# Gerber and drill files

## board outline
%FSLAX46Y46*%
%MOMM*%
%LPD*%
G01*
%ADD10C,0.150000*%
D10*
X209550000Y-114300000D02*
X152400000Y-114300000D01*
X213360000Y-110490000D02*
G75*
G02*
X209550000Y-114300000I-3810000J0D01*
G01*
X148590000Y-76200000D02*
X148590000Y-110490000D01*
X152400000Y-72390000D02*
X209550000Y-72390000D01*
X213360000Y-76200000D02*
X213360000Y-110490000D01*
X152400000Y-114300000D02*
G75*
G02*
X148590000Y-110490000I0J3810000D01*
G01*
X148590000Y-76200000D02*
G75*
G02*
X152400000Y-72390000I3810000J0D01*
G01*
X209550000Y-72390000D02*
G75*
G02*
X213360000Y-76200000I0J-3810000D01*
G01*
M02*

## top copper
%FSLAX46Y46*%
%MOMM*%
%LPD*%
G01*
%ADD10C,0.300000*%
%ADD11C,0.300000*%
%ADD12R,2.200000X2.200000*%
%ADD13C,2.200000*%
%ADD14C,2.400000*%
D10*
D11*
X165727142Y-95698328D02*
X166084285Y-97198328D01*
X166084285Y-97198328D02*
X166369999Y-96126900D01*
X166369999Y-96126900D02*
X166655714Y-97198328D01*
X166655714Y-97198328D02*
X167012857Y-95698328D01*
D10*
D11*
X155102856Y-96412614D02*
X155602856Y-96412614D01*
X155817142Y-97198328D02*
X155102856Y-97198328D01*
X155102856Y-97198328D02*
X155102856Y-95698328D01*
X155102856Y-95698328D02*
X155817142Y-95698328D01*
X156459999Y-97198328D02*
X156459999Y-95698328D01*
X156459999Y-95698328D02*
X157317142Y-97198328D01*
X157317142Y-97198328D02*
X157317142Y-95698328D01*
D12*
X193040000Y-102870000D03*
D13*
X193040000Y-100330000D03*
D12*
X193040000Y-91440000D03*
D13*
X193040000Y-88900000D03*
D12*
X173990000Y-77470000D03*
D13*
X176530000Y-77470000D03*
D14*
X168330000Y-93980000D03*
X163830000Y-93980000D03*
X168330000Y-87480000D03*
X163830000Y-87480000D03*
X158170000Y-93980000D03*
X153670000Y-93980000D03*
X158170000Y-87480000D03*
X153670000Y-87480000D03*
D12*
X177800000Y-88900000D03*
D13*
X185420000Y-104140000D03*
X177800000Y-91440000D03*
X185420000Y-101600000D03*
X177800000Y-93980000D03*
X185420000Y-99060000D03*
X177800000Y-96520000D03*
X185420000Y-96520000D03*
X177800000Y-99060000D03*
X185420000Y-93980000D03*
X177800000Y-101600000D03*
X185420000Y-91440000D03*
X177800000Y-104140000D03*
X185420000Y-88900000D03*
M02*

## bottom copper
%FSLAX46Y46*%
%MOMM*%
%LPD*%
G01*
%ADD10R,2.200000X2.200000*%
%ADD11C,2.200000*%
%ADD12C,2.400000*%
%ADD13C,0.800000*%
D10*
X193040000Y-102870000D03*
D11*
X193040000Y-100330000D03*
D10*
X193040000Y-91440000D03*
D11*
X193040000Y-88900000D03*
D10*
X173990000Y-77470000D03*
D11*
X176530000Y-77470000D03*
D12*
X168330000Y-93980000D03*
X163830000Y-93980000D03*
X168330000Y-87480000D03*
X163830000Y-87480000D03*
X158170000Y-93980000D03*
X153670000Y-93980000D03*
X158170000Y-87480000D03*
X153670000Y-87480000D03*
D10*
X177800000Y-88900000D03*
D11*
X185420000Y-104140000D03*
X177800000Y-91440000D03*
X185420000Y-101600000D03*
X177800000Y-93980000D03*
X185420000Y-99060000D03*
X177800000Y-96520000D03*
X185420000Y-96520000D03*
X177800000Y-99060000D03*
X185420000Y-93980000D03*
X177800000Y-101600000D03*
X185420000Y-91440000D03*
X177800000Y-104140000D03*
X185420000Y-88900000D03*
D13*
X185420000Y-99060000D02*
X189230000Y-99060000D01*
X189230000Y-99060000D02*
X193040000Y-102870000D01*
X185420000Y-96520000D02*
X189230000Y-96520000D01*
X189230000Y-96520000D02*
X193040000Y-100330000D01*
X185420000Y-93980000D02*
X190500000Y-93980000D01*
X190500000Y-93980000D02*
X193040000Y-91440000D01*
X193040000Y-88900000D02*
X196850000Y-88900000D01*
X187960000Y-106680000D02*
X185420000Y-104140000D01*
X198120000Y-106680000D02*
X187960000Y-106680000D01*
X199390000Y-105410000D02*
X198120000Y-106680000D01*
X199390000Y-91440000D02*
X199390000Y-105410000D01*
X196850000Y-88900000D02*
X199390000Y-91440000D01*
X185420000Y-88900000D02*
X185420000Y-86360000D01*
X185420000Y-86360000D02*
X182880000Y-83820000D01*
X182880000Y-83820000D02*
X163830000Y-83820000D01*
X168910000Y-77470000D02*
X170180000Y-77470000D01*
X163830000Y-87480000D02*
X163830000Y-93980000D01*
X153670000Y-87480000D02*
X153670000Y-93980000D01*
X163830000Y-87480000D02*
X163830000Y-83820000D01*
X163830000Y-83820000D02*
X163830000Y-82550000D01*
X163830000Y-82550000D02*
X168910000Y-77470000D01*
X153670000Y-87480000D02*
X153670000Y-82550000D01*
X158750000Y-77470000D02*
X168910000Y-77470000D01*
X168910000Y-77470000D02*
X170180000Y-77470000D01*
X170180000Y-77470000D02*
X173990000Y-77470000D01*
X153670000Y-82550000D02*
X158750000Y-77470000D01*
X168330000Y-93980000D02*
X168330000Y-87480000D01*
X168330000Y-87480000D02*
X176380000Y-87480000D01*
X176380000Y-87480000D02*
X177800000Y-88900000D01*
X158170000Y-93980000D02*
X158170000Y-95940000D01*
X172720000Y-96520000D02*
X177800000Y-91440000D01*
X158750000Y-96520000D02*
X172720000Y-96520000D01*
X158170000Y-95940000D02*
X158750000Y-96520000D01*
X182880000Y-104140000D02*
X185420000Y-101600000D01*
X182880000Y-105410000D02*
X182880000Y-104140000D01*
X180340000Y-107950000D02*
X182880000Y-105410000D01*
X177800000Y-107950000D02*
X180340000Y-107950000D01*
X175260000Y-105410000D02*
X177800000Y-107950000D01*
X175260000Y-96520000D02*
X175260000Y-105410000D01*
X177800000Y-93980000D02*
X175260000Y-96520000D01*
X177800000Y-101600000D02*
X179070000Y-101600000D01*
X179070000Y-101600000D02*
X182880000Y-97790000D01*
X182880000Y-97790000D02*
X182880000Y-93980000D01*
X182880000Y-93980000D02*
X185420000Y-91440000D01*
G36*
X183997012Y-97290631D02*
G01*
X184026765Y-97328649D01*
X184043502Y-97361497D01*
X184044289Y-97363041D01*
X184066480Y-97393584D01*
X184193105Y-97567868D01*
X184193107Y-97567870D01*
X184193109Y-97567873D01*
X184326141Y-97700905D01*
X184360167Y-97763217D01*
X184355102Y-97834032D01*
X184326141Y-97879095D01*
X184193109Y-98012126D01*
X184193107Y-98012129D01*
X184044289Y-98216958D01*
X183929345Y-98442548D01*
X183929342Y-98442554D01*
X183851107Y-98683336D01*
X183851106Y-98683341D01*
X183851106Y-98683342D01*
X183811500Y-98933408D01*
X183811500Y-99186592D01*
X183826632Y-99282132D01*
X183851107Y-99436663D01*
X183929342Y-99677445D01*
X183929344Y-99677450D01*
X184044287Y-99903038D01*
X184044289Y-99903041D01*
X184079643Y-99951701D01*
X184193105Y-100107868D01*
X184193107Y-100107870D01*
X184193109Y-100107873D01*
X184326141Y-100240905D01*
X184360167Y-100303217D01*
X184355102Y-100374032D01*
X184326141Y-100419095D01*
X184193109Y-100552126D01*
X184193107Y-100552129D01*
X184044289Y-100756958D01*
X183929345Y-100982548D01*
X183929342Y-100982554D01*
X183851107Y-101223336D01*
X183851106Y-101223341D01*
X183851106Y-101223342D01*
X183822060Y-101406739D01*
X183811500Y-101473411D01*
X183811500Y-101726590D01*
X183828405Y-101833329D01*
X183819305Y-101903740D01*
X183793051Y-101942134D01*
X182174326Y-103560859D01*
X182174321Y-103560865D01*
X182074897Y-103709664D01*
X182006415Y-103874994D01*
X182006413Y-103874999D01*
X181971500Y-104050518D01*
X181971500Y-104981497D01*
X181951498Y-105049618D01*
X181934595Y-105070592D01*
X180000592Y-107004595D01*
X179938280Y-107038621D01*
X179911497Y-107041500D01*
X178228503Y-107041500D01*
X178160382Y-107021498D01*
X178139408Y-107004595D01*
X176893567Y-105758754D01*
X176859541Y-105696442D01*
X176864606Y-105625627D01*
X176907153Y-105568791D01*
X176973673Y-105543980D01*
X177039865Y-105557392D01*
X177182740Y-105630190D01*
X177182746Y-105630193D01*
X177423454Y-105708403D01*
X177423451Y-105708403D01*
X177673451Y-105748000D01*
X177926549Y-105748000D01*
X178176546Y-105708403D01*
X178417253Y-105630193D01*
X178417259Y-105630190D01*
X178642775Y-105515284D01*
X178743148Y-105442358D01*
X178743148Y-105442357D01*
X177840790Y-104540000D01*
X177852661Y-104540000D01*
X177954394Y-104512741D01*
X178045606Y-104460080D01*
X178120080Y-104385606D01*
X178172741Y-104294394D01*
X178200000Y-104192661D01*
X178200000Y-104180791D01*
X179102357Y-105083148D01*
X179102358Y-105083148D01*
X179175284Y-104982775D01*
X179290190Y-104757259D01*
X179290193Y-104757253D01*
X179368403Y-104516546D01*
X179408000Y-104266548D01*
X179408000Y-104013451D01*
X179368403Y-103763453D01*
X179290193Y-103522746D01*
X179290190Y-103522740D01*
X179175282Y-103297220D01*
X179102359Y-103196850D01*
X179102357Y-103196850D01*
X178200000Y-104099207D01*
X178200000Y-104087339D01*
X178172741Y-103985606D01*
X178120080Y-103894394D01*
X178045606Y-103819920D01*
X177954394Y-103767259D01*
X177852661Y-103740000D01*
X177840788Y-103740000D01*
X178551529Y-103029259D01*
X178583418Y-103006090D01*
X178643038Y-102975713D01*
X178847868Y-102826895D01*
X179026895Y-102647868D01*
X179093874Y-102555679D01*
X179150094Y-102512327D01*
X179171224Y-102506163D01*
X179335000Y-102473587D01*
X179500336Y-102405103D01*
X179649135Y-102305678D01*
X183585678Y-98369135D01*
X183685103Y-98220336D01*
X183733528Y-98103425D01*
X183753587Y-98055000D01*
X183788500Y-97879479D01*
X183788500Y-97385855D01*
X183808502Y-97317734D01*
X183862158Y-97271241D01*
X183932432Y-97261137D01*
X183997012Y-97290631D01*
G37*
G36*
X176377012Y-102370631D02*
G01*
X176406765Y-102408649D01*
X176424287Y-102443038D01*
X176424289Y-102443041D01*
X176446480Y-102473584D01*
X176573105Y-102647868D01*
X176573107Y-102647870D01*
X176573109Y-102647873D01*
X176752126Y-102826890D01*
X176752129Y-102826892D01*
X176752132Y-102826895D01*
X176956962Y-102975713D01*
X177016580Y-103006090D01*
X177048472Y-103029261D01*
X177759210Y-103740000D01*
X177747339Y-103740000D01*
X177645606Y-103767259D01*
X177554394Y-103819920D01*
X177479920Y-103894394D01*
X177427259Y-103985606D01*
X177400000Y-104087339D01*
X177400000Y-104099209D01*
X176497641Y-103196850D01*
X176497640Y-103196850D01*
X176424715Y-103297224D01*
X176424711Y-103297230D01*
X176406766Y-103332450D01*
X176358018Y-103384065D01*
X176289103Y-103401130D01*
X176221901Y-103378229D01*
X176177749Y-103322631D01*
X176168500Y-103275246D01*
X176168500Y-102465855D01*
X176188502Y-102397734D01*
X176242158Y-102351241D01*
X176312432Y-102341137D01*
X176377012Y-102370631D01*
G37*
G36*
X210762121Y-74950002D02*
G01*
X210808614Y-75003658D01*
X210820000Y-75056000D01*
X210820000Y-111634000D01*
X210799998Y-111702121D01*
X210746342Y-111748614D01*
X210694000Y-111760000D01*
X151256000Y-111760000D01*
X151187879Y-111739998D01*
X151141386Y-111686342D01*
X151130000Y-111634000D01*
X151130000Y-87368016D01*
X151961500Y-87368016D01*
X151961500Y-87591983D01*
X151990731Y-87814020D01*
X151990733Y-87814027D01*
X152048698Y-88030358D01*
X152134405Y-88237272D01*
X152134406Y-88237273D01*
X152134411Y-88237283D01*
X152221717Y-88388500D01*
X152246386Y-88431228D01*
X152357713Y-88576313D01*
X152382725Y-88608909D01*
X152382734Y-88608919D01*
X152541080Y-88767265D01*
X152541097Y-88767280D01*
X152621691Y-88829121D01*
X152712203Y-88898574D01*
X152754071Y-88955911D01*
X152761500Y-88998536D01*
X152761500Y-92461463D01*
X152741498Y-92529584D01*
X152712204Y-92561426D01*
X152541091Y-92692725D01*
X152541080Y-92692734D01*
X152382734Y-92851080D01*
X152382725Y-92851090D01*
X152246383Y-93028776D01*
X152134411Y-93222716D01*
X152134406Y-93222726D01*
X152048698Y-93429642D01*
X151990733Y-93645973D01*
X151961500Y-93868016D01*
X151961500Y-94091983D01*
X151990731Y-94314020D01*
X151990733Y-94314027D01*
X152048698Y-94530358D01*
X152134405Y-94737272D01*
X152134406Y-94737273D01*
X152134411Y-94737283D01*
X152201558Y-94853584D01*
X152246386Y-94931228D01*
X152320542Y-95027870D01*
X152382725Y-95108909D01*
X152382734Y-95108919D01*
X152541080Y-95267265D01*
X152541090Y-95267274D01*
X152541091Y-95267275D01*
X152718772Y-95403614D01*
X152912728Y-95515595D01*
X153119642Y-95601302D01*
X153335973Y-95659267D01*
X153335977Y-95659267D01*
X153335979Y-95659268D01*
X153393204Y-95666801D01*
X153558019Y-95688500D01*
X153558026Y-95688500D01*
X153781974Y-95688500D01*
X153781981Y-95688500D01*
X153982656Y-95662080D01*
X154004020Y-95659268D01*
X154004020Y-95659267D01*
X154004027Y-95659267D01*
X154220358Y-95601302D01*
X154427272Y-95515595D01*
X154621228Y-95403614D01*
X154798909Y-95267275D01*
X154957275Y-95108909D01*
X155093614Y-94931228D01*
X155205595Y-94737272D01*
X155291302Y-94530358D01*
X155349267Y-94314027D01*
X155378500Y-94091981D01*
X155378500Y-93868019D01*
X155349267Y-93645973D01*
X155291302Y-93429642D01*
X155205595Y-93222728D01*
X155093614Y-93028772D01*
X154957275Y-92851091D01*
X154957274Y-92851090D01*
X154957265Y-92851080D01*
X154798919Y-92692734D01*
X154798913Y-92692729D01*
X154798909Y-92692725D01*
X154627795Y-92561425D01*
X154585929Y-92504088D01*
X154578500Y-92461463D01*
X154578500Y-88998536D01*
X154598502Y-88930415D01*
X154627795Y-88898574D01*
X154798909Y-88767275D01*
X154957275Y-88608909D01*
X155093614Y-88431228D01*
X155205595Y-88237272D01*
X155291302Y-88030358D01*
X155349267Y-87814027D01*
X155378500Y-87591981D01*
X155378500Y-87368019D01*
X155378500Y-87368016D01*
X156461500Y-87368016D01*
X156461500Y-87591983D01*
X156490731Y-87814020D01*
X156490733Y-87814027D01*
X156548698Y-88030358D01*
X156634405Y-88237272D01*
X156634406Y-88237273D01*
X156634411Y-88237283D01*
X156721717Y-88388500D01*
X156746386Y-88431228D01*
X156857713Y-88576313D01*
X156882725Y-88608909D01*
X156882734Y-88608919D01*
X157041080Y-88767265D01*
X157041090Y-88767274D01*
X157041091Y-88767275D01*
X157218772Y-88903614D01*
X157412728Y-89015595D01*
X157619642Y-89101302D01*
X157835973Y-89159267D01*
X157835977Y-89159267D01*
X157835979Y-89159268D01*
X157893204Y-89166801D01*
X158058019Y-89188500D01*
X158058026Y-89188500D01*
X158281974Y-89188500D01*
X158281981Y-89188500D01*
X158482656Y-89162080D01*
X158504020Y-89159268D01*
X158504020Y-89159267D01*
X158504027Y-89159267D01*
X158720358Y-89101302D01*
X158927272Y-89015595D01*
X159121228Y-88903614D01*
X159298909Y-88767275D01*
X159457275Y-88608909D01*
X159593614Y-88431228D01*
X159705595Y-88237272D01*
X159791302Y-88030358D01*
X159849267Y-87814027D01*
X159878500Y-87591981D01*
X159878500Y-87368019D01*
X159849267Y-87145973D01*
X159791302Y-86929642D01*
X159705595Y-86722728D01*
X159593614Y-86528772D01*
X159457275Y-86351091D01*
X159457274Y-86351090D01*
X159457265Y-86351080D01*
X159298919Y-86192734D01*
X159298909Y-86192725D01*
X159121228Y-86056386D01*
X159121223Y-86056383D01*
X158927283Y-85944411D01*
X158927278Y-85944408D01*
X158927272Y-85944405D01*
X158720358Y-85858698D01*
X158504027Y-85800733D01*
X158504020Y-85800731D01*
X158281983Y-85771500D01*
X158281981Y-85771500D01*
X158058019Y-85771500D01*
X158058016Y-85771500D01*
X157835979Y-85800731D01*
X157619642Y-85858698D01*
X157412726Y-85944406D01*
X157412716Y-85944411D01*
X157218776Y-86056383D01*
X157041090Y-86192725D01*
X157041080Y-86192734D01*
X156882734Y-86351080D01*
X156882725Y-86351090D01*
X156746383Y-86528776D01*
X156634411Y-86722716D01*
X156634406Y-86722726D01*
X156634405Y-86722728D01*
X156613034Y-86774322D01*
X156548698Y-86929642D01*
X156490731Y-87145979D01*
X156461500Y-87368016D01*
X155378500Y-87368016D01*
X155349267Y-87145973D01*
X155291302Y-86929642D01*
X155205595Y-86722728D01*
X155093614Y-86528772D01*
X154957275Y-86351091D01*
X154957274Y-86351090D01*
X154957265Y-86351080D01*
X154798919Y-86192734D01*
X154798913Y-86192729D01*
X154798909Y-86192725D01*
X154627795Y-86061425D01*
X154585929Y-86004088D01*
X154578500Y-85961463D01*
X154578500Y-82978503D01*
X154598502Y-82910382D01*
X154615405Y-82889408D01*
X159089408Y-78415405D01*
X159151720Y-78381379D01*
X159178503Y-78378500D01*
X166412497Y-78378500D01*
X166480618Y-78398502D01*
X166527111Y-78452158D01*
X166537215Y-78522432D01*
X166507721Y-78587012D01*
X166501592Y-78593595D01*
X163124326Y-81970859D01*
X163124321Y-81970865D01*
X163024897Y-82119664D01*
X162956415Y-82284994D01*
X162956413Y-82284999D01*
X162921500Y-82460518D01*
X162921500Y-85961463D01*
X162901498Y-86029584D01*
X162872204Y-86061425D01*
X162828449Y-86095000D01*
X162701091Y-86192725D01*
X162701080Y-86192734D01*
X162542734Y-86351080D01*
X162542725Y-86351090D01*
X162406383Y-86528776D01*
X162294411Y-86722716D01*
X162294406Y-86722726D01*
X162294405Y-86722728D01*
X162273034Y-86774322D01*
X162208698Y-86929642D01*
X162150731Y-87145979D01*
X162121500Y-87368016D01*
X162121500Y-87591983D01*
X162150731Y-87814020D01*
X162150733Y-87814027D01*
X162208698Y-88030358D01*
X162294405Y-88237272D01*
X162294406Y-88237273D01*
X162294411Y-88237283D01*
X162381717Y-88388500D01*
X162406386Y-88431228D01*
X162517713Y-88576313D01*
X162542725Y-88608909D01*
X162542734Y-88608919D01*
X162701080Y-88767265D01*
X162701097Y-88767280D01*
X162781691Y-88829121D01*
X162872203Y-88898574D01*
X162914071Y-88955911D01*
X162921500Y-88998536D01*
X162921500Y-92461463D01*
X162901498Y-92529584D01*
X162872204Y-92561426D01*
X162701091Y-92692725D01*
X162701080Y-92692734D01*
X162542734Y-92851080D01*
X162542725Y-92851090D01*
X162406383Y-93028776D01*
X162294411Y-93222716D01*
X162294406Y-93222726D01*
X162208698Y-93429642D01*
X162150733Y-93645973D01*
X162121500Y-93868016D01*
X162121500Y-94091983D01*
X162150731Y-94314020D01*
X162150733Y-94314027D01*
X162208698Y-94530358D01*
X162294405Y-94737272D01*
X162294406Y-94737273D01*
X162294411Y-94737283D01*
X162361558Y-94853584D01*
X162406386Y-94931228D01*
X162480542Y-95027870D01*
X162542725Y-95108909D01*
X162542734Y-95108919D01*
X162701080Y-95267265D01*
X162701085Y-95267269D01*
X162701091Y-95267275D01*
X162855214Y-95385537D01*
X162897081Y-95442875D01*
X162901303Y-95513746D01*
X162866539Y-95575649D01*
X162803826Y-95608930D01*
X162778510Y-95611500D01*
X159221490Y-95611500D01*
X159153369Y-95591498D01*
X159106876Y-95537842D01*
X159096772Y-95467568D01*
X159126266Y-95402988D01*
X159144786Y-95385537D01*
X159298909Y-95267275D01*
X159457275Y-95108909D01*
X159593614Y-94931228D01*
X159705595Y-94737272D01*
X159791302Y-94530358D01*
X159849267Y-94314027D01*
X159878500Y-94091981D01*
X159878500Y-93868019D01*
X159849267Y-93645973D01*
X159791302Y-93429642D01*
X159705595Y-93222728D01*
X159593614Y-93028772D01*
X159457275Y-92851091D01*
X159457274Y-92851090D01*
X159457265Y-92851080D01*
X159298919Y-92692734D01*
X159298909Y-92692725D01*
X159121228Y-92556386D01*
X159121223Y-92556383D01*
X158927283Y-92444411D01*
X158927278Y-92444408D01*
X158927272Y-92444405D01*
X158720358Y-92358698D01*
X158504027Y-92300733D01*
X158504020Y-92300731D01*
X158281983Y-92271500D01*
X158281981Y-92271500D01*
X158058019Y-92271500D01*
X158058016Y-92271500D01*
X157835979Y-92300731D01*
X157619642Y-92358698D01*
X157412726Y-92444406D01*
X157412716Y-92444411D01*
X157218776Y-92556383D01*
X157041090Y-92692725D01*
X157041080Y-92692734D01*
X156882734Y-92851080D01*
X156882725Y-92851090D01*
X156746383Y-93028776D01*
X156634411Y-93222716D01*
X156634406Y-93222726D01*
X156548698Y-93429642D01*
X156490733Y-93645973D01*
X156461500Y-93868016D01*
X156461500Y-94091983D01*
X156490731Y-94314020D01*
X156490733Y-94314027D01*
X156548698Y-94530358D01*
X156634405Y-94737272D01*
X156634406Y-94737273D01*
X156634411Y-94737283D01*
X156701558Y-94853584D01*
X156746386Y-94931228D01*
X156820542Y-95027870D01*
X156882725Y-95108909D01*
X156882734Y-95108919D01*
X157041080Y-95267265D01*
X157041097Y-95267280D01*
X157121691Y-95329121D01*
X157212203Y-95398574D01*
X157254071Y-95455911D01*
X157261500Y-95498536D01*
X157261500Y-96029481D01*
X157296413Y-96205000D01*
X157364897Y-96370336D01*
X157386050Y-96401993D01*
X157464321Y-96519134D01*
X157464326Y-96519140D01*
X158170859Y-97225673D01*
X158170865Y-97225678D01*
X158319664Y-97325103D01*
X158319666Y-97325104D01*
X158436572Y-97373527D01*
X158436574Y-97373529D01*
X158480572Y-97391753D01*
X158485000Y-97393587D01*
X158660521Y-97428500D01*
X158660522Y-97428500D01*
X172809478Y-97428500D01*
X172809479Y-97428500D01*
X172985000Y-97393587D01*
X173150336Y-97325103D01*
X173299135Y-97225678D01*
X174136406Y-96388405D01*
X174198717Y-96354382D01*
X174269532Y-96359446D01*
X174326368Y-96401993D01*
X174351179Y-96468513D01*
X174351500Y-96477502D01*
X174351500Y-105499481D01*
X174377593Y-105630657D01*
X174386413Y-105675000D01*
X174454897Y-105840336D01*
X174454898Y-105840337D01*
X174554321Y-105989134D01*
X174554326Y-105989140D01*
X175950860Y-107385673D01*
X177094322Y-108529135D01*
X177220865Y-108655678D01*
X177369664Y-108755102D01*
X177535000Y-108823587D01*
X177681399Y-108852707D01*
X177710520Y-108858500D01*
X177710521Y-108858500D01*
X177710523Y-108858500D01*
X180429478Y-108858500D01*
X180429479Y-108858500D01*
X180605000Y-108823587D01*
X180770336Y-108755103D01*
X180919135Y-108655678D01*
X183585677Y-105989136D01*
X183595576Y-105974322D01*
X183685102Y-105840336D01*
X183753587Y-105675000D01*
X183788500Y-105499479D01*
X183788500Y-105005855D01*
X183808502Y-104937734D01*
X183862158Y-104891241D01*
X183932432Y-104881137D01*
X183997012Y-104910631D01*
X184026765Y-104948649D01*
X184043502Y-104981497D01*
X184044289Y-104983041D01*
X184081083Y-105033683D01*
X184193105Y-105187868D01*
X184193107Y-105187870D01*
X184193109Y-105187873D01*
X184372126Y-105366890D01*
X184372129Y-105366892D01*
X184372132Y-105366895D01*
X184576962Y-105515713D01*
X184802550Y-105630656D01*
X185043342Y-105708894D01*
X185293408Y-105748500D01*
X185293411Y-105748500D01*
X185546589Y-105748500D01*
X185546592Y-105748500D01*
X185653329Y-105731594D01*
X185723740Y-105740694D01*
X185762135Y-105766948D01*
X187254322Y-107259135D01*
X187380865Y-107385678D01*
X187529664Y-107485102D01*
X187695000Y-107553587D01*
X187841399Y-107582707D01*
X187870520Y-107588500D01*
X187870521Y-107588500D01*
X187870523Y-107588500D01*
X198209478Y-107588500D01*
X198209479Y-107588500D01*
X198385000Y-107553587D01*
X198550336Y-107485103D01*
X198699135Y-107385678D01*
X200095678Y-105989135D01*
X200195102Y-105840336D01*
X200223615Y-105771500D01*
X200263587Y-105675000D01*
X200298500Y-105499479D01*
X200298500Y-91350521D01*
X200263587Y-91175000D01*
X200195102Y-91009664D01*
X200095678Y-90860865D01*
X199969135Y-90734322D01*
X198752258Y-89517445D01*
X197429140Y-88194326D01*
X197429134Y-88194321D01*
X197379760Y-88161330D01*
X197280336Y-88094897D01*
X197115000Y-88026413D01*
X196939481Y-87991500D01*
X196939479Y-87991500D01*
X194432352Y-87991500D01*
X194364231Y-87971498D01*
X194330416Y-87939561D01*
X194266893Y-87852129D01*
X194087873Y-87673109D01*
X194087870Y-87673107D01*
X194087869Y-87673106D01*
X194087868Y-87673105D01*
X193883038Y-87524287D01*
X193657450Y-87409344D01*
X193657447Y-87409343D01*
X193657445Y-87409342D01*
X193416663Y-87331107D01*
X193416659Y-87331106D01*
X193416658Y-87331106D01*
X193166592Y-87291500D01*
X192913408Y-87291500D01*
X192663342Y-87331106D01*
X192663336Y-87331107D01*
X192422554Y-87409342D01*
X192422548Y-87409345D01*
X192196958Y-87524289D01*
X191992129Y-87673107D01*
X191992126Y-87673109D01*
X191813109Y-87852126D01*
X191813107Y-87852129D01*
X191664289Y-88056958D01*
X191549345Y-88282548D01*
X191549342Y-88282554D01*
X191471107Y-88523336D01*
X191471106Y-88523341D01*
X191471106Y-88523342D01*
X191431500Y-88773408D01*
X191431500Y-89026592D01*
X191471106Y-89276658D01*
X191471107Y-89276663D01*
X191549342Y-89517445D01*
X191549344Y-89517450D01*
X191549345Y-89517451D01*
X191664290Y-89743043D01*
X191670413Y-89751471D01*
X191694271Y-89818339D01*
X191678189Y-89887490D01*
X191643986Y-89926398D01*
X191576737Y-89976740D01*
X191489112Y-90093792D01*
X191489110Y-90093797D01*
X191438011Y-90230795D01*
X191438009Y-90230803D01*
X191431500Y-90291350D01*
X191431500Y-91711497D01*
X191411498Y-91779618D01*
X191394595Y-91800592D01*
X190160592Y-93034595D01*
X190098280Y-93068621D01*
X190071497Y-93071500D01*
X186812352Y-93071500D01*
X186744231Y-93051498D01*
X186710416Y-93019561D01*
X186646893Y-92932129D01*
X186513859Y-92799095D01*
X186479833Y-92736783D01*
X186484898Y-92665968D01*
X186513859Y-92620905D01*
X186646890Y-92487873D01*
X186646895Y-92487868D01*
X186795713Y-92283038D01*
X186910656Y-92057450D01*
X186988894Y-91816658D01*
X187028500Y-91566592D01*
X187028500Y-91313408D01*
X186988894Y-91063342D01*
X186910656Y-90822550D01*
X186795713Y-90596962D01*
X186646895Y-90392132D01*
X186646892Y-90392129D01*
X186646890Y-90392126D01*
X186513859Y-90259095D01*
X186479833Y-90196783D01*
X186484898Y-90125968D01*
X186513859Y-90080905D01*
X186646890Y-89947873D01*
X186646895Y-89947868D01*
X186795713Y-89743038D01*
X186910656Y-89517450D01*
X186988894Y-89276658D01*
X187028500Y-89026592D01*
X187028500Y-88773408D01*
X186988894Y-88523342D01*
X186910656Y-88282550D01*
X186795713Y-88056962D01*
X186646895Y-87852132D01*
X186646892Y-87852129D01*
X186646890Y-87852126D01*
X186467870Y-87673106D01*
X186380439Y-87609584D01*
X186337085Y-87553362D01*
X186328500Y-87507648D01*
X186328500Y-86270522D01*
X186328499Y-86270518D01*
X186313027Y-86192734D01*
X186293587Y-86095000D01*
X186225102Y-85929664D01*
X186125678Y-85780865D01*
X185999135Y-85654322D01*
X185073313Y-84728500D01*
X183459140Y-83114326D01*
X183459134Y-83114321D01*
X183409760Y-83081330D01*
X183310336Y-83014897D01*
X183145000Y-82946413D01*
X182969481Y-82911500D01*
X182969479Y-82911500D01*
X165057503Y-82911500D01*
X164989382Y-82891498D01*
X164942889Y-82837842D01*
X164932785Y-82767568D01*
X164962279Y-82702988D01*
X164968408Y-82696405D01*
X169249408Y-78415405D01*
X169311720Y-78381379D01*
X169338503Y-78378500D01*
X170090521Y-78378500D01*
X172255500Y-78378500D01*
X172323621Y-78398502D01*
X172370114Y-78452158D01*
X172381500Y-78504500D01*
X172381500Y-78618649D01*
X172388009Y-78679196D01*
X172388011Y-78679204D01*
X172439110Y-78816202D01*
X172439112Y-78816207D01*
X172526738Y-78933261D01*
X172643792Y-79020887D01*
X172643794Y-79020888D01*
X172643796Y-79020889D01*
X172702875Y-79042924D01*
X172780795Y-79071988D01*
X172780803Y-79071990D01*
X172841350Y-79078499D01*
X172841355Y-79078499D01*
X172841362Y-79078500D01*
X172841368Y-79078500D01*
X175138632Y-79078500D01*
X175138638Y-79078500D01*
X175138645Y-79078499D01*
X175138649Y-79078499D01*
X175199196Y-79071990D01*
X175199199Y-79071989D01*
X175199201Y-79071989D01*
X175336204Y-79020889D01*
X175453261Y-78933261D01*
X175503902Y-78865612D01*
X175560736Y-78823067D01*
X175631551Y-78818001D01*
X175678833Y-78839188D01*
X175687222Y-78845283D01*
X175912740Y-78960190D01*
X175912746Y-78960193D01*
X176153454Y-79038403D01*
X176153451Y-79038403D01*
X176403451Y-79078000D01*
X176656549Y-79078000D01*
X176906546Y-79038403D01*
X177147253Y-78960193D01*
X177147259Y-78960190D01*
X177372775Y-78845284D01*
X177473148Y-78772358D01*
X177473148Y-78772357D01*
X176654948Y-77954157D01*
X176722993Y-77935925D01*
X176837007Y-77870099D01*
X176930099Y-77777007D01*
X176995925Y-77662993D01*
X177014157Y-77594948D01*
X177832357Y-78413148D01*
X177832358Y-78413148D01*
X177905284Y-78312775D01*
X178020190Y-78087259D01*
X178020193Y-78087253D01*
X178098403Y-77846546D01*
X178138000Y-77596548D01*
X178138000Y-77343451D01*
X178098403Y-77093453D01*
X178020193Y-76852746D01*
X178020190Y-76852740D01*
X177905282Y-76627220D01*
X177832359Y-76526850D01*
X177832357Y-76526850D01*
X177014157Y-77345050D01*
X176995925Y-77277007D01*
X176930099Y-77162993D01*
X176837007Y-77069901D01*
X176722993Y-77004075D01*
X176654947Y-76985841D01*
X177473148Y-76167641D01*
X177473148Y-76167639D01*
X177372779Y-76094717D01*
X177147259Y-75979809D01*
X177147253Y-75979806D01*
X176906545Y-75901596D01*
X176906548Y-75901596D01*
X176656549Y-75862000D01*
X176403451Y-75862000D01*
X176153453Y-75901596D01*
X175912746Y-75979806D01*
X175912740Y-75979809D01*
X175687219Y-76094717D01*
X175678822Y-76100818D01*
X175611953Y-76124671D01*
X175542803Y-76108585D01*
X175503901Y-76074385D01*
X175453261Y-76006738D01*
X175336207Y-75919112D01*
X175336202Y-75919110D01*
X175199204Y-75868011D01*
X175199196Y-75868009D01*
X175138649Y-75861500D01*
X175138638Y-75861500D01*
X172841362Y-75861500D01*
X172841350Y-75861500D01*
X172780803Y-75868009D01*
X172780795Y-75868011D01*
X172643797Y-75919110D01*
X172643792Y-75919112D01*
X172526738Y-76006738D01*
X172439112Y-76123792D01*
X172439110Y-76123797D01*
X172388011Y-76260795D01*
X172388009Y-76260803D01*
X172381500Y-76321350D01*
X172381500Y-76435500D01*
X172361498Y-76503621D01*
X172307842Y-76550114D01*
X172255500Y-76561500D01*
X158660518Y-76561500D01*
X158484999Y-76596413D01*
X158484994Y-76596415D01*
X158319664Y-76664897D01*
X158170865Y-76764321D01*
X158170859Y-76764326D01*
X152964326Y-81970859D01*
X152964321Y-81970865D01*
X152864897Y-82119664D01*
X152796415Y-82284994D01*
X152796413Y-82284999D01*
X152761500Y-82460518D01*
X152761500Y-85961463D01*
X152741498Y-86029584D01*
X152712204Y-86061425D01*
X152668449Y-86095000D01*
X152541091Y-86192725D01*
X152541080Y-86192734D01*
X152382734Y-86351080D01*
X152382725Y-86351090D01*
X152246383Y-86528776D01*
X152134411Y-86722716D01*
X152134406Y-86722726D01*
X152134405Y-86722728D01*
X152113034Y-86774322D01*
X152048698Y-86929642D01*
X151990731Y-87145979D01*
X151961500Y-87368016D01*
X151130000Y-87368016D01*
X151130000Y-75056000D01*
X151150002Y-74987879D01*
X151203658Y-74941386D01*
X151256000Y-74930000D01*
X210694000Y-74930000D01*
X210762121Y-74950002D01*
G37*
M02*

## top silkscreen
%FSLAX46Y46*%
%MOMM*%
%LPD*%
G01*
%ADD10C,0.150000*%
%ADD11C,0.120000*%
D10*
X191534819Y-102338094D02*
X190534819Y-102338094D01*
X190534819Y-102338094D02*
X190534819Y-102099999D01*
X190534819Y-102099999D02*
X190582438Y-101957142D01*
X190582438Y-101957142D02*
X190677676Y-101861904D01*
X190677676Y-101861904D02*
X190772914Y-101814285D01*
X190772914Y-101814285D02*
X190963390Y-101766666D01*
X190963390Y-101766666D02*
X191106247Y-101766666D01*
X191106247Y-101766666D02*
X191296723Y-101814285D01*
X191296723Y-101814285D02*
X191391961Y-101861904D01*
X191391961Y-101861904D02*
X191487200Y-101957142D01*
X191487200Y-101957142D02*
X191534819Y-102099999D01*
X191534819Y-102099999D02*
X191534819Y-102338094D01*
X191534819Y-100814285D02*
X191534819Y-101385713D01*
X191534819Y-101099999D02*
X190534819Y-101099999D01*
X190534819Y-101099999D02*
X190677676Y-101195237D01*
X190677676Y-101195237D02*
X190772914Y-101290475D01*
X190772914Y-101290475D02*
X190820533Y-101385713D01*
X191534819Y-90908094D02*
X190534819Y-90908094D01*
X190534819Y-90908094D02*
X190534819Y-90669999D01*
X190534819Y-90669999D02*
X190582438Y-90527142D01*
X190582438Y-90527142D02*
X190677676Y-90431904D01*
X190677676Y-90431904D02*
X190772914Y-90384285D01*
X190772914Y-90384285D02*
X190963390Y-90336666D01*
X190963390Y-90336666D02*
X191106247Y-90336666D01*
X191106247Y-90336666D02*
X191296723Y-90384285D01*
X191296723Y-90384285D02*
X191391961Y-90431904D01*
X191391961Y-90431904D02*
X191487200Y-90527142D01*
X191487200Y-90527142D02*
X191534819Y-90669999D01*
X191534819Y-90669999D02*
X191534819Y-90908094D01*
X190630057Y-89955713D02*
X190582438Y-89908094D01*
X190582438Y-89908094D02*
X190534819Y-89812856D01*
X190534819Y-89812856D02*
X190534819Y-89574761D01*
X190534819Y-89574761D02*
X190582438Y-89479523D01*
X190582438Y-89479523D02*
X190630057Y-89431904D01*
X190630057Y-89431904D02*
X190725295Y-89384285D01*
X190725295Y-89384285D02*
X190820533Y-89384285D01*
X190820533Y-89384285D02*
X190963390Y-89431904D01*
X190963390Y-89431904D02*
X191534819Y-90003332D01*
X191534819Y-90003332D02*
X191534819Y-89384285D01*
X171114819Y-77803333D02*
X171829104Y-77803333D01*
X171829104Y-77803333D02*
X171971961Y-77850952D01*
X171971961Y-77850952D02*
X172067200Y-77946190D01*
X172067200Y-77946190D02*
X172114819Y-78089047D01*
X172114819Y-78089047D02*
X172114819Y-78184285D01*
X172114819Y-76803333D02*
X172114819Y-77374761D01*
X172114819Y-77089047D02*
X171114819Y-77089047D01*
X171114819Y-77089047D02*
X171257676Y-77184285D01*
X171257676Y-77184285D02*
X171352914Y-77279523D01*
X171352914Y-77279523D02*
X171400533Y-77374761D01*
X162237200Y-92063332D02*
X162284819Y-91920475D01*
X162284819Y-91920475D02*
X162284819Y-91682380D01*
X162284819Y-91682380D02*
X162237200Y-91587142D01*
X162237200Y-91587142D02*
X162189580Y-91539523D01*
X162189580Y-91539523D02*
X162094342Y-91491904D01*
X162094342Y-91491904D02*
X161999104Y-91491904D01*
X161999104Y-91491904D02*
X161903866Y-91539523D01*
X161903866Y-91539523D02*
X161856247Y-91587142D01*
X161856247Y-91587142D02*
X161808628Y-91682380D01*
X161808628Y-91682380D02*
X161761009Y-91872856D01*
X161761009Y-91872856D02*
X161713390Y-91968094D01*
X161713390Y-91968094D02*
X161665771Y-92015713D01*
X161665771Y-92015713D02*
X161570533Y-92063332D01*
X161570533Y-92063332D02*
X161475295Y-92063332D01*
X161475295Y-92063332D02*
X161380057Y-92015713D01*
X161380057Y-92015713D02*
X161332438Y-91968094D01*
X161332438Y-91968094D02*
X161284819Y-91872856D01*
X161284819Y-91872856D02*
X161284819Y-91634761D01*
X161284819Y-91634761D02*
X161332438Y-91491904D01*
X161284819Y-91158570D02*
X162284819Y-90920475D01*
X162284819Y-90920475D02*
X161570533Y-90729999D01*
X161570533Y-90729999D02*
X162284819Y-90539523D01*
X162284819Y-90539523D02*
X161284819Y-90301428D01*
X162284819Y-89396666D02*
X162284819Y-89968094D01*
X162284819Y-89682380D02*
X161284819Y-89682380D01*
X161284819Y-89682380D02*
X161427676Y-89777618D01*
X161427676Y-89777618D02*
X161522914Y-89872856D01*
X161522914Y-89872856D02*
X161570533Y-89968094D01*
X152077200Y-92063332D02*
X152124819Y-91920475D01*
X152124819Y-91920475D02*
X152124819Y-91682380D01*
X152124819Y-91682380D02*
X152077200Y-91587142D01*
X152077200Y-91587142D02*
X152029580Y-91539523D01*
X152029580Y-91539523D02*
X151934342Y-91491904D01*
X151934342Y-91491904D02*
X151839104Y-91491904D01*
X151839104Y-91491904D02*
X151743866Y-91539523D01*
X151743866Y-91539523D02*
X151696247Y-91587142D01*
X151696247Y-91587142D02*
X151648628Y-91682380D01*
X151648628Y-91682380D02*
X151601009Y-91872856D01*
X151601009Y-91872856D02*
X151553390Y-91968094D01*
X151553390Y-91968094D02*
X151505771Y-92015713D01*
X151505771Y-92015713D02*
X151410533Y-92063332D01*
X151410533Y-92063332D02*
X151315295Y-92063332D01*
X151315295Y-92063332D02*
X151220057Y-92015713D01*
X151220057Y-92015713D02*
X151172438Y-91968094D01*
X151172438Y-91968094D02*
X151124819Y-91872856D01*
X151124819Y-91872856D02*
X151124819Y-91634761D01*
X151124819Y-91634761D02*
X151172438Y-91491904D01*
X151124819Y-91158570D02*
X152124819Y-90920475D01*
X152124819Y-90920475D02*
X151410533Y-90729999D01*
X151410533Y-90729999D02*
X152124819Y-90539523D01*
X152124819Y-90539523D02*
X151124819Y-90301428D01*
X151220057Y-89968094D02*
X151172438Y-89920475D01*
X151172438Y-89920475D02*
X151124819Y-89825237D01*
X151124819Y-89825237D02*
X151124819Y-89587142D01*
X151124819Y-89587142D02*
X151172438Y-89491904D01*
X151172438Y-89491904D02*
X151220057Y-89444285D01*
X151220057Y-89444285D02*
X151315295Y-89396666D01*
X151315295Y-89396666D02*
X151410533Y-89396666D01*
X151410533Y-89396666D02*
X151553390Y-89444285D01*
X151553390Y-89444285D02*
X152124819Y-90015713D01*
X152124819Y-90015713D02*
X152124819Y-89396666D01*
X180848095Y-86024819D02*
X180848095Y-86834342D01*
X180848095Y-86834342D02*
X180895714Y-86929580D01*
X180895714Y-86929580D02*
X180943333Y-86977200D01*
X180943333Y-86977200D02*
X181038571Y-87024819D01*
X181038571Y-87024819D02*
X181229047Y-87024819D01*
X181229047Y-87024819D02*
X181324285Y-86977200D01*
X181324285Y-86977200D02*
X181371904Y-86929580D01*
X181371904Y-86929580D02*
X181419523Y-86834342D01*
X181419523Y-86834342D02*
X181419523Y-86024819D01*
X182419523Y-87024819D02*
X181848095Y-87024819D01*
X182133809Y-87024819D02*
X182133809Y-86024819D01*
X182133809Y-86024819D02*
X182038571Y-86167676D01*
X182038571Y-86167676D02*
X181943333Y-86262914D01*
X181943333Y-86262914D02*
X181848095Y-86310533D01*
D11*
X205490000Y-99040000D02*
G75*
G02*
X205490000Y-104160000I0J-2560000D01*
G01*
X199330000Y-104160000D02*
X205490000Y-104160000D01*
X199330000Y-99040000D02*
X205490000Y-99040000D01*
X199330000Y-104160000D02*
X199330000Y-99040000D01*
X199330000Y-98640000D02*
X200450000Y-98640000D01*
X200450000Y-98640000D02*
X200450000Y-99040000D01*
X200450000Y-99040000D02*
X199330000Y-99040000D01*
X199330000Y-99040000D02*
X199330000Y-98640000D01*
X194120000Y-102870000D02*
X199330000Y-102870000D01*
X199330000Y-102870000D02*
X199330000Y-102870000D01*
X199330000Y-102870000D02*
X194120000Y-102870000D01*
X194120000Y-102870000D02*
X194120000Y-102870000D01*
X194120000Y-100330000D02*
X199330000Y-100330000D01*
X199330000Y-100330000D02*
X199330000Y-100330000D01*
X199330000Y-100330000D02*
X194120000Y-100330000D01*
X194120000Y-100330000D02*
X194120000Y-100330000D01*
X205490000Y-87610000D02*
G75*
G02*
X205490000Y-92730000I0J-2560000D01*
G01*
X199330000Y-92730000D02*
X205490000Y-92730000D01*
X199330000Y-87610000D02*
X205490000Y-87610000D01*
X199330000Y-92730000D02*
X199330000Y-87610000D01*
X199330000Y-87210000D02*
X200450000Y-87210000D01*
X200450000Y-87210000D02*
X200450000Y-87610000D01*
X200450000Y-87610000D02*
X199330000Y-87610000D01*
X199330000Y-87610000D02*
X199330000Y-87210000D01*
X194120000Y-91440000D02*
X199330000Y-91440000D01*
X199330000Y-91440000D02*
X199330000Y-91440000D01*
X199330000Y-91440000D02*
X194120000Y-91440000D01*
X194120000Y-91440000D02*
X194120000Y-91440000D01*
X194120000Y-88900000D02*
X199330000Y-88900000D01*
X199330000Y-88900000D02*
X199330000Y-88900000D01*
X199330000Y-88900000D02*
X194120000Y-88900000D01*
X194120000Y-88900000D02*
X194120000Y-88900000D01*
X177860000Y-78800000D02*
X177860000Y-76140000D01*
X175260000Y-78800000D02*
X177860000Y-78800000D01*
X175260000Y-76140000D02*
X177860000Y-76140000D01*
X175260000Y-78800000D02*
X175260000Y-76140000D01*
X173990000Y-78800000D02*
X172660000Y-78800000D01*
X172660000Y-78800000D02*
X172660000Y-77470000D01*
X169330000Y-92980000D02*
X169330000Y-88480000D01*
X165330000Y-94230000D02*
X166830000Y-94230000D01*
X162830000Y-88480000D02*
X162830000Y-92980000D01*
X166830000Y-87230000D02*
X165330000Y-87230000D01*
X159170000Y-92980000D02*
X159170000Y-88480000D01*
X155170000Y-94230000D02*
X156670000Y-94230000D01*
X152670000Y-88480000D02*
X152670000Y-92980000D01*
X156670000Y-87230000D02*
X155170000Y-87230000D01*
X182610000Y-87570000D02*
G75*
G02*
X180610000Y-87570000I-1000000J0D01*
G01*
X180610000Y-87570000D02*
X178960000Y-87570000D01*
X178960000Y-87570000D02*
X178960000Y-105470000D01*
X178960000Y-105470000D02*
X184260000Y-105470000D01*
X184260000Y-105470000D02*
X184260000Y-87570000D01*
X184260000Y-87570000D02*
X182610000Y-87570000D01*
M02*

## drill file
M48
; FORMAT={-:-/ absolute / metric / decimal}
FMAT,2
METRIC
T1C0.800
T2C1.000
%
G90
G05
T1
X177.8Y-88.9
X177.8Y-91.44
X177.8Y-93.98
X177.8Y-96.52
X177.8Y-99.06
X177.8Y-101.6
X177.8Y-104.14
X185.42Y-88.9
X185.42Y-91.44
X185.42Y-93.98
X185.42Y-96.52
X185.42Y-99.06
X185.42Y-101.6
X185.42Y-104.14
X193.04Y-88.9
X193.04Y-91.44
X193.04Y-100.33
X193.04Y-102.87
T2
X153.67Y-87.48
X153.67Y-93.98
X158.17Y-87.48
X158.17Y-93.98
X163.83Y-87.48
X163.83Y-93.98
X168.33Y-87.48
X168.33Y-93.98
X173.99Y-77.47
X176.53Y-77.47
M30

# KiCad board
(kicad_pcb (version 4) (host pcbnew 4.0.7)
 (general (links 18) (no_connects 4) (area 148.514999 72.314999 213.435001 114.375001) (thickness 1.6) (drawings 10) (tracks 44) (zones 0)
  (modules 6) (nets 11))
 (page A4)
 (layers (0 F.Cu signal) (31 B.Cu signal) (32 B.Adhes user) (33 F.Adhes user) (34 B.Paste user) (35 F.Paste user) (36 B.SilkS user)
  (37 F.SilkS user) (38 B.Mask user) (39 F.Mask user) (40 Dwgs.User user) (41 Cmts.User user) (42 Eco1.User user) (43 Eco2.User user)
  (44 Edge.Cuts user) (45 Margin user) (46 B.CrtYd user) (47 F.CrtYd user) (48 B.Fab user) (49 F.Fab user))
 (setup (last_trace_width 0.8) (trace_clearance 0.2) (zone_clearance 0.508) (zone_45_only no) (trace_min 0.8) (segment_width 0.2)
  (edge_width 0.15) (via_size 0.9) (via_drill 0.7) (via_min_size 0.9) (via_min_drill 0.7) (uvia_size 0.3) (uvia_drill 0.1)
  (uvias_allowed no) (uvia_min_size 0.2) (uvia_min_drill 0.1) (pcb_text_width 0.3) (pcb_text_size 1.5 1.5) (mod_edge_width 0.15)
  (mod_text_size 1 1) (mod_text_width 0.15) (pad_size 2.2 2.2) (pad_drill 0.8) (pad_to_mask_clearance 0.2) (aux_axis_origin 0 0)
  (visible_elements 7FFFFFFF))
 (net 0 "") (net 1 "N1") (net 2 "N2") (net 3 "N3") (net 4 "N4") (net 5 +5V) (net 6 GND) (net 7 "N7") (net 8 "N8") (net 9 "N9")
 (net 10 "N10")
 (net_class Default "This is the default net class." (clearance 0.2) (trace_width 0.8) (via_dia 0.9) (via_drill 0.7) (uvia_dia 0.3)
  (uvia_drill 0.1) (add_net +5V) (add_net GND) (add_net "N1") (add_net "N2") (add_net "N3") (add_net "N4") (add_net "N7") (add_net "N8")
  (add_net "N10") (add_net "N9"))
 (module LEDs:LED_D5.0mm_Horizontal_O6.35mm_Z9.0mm (layer F.Cu) (at 193.04 102.87 90)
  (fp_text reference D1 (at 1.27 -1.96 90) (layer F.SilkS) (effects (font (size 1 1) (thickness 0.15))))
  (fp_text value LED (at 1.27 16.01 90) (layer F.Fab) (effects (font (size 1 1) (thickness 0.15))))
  (fp_arc (start 1.27 12.45) (end -1.29 12.45) (angle -180) (layer F.SilkS) (width 0.12))
  (fp_line (start -1.29 6.29) (end -1.29 12.45) (layer F.SilkS) (width 0.12))
  (fp_line (start 3.83 6.29) (end 3.83 12.45) (layer F.SilkS) (width 0.12))
  (fp_line (start -1.29 6.29) (end 3.83 6.29) (layer F.SilkS) (width 0.12))
  (fp_line (start 4.23 6.29) (end 4.23 7.41) (layer F.SilkS) (width 0.12))
  (fp_line (start 4.23 7.41) (end 3.83 7.41) (layer F.SilkS) (width 0.12))
  (fp_line (start 3.83 7.41) (end 3.83 6.29) (layer F.SilkS) (width 0.12))
  (fp_line (start 3.83 6.29) (end 4.23 6.29) (layer F.SilkS) (width 0.12))
  (fp_line (start 0 1.08) (end 0 6.29) (layer F.SilkS) (width 0.12))
  (fp_line (start 0 6.29) (end 0 6.29) (layer F.SilkS) (width 0.12))
  (fp_line (start 0 6.29) (end 0 1.08) (layer F.SilkS) (width 0.12))
  (fp_line (start 0 1.08) (end 0 1.08) (layer F.SilkS) (width 0.12))
  (fp_line (start 2.54 1.08) (end 2.54 6.29) (layer F.SilkS) (width 0.12))
  (fp_line (start 2.54 6.29) (end 2.54 6.29) (layer F.SilkS) (width 0.12))
  (fp_line (start 2.54 6.29) (end 2.54 1.08) (layer F.SilkS) (width 0.12))
  (fp_line (start 2.54 1.08) (end 2.54 1.08) (layer F.SilkS) (width 0.12))
  (pad 1 thru_hole rect (at 0 0 90) (size 2.2 2.2) (drill 0.8) (layers *.Cu *.Mask) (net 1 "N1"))
  (pad 2 thru_hole circle (at 2.54 0 90) (size 2.2 2.2) (drill 0.8) (layers *.Cu *.Mask) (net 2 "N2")))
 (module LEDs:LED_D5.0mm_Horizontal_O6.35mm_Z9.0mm (layer F.Cu) (at 193.04 91.44 90)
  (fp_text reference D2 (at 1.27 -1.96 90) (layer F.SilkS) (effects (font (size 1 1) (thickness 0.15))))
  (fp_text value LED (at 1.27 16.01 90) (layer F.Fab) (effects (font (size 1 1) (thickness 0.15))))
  (fp_arc (start 1.27 12.45) (end -1.29 12.45) (angle -180) (layer F.SilkS) (width 0.12))
  (fp_line (start -1.29 6.29) (end -1.29 12.45) (layer F.SilkS) (width 0.12))
  (fp_line (start 3.83 6.29) (end 3.83 12.45) (layer F.SilkS) (width 0.12))
  (fp_line (start -1.29 6.29) (end 3.83 6.29) (layer F.SilkS) (width 0.12))
  (fp_line (start 4.23 6.29) (end 4.23 7.41) (layer F.SilkS) (width 0.12))
  (fp_line (start 4.23 7.41) (end 3.83 7.41) (layer F.SilkS) (width 0.12))
  (fp_line (start 3.83 7.41) (end 3.83 6.29) (layer F.SilkS) (width 0.12))
  (fp_line (start 3.83 6.29) (end 4.23 6.29) (layer F.SilkS) (width 0.12))
  (fp_line (start 0 1.08) (end 0 6.29) (layer F.SilkS) (width 0.12))
  (fp_line (start 0 6.29) (end 0 6.29) (layer F.SilkS) (width 0.12))
  (fp_line (start 0 6.29) (end 0 1.08) (layer F.SilkS) (width 0.12))
  (fp_line (start 0 1.08) (end 0 1.08) (layer F.SilkS) (width 0.12))
  (fp_line (start 2.54 1.08) (end 2.54 6.29) (layer F.SilkS) (width 0.12))
  (fp_line (start 2.54 6.29) (end 2.54 6.29) (layer F.SilkS) (width 0.12))
  (fp_line (start 2.54 6.29) (end 2.54 1.08) (layer F.SilkS) (width 0.12))
  (fp_line (start 2.54 1.08) (end 2.54 1.08) (layer F.SilkS) (width 0.12))
  (pad e1 thru_hole rect (at 0 0 90) (size 2.2 2.2) (drill 0.8) (layers *.Cu *.Mask) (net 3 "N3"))
  (pad 2 thru_hole circle (at 2.54 0 90) (size 2.2 2.2) (drill 0.8) (layers *.Cu *.Mask) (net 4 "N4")))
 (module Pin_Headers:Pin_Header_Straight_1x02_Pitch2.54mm (layer F.Cu) (at 173.99 77.47 90)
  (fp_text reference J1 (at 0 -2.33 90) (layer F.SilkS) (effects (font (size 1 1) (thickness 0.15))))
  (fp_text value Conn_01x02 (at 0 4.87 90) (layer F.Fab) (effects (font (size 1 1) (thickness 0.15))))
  (fp_line (start -1.33 3.87) (end 1.33 3.87) (layer F.SilkS) (width 0.12))
  (fp_line (start -1.33 1.27) (end -1.33 3.87) (layer F.SilkS) (width 0.12))
  (fp_line (start 1.33 1.27) (end 1.33 3.87) (layer F.SilkS) (width 0.12))
  (fp_line (start -1.33 1.27) (end 1.33 1.27) (layer F.SilkS) (width 0.12))
  (fp_line (start -1.33 0) (end -1.33 -1.33) (layer F.SilkS) (width 0.12))
  (fp_line (start -1.33 -1.33) (end 0 -1.33) (layer F.SilkS) (width 0.12))
  (pad 1 thru_hole rect (at 0 0 90) (size 2.2 2.2) (drill 1) (layers *.Cu *.Mask) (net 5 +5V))
  (pad e2 thru_hole circle (at 0 2.54 90) (size 2.2 2.2) (drill 1) (layers *.Cu *.Mask) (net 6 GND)))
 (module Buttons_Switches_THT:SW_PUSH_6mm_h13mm (layer F.Cu) (at 163.83 93.98 90)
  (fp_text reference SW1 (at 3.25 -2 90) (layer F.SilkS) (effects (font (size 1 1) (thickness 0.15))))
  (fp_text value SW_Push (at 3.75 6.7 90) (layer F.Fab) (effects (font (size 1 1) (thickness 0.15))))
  (fp_line (start 1 5.5) (end 5.5 5.5) (layer F.SilkS) (width 0.12))
  (fp_line (start -0.25 1.5) (end -0.25 3) (layer F.SilkS) (width 0.12))
  (fp_line (start 5.5 -1) (end 1 -1) (layer F.SilkS) (width 0.12))
  (fp_line (start 6.75 3) (end 6.75 1.5) (layer F.SilkS) (width 0.12))
  (pad 2 thru_hole circle (at 0 4.5 180) (size 2.4 2.4) (drill 1) (layers *.Cu *.Mask) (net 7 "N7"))
  (pad 1 thru_hole circle (at 0 0 180) (size 2.4 2.4) (drill 1) (layers *.Cu *.Mask) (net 5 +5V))
  (pad 2 thru_hole circle (at 6.5 4.5 180) (size 2.4 2.4) (drill 1) (layers *.Cu *.Mask) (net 7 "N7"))
  (pad 1 thru_hole circle (at 6.5 0 180) (size 2.4 2.4) (drill 1) (layers *.Cu *.Mask) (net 5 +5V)))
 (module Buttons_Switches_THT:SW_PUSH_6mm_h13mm (layer F.Cu) (at 153.67 93.98 90)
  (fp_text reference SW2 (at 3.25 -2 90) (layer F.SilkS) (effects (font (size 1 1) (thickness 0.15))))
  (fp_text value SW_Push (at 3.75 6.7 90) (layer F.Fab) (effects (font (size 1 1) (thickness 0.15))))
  (fp_line (start 1 5.5) (end 5.5 5.5) (layer F.SilkS) (width 0.12))
  (fp_line (start -0.25 1.5) (end -0.25 3) (layer F.SilkS) (width 0.12))
  (fp_line (start 5.5 -1) (end 1 -1) (layer F.SilkS) (width 0.12))
  (fp_line (start 6.75 3) (end 6.75 1.5) (layer F.SilkS) (width 0.12))
  (pad 2 thru_hole circle (at 0 4.5 180) (size 2.4 2.4) (drill 1) (layers *.Cu *.Mask) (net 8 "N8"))
  (pad 1 thru_hole circle (at 0 0 180) (size 2.4 2.4) (drill 1) (layers *.Cu *.Mask) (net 5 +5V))
  (pad 2 thru_hole circle (at 6.5 4.5 180) (size 2.4 2.4) (drill 1) (layers *.Cu *.Mask) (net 8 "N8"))
  (pad 1 thru_hole circle (at 6.5 0 180) (size 2.4 2.4) (drill 1) (layers *.Cu *.Mask) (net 5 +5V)))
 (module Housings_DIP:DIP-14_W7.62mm (layer F.Cu) (at 177.8 88.9)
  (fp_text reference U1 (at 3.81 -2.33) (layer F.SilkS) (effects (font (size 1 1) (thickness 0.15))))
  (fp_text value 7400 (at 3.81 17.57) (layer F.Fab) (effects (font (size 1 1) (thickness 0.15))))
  (fp_arc (start 3.81 -1.33) (end 2.81 -1.33) (angle -180) (layer F.SilkS) (width 0.12))
  (fp_line (start 2.81 -1.33) (end 1.16 -1.33) (layer F.SilkS) (width 0.12))
  (fp_line (start 1.16 -1.33) (end 1.16 16.57) (layer F.SilkS) (width 0.12))
  (fp_line (start 1.16 16.57) (end 6.46 16.57) (layer F.SilkS) (width 0.12))
  (fp_line (start 6.46 16.57) (end 6.46 -1.33) (layer F.SilkS) (width 0.12))
  (fp_line (start 6.46 -1.33) (end 4.81 -1.33) (layer F.SilkS) (width 0.12))
  (pad 1 thru_hole rect (at 0 0) (size 2.2 2.2) (drill 0.8) (layers *.Cu *.Mask) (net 7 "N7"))
  (pad 8 thru_hole circle (at 7.62 15.24) (size 2.2 2.2) (drill 0.8) (layers *.Cu *.Mask) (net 4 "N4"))
  (pad 2 thru_hole circle (at 0 2.54) (size 2.2 2.2) (drill 0.8) (layers *.Cu *.Mask) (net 8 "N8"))
  (pad 9 thru_hole circle (at 7.62 12.7) (size 2.2 2.2) (drill 0.8) (layers *.Cu *.Mask) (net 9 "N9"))
  (pad 3 thru_hole circle (at 0 5.08) (size 2.2 2.2) (drill 0.8) (layers *.Cu *.Mask) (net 9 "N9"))
  (pad 10 thru_hole circle (at 7.62 10.16) (size 2.2 2.2) (drill 0.8) (layers *.Cu *.Mask) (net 1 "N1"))
  (pad 4 thru_hole circle (at 0 7.62) (size 2.2 2.2) (drill 0.8) (layers *.Cu *.Mask) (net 8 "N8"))
  (pad 11 thru_hole circle (at 7.62 7.62) (size 2.2 2.2) (drill 0.8) (layers *.Cu *.Mask) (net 2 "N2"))
  (pad 5 thru_hole circle (at 0 10.16) (size 2.2 2.2) (drill 0.8) (layers *.Cu *.Mask) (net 7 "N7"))
  (pad 12 thru_hole circle (at 7.62 5.08) (size 2.2 2.2) (drill 0.8) (layers *.Cu *.Mask) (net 3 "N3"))
  (pad 6 thru_hole circle (at 0 12.7) (size 2.2 2.2) (drill 0.8) (layers *.Cu *.Mask) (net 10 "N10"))
  (pad 13 thru_hole circle (at 7.62 2.54) (size 2.2 2.2) (drill 0.8) (layers *.Cu *.Mask) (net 10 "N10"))
  (pad 7 thru_hole circle (at 0 15.24) (size 2.2 2.2) (drill 0.8) (layers *.Cu *.Mask) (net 6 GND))
  (pad 14 thru_hole circle (at 7.62 0) (size 2.2 2.2) (drill 0.8) (layers *.Cu *.Mask) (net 5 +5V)))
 (gr_line (start 209.55 114.3) (end 152.4 114.3) (angle 90) (layer Edge.Cuts) (width 0.15))
 (gr_arc (start 209.55 110.49) (end 213.36 110.49) (angle 90) (layer Edge.Cuts) (width 0.15))
 (gr_line (start 148.59 76.2) (end 148.59 110.49) (angle 90) (layer Edge.Cuts) (width 0.15))
 (gr_line (start 152.4 72.39) (end 209.55 72.39) (angle 90) (layer Edge.Cuts) (width 0.15))
 (gr_line (start 213.36 76.2) (end 213.36 110.49) (angle 90) (layer Edge.Cuts) (width 0.15))
 (gr_arc (start 152.4 110.49) (end 152.4 114.3) (angle 90) (layer Edge.Cuts) (width 0.15))
 (gr_arc (start 152.4 76.2) (end 148.59 76.2) (angle 90) (layer Edge.Cuts) (width 0.15))
 (gr_arc (start 209.55 76.2) (end 209.55 72.39) (angle 90) (layer Edge.Cuts) (width 0.15))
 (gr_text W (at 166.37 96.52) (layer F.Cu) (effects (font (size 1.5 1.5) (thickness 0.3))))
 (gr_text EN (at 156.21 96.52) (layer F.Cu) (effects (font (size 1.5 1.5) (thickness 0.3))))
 (segment (start 185.42 99.06) (end 189.23 99.06) (width 0.8) (layer B.Cu) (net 1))
 (segment (start 189.23 99.06) (end 193.04 102.87) (width 0.8) (layer B.Cu) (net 1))
 (segment (start 185.42 96.52) (end 189.23 96.52) (width 0.8) (layer B.Cu) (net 2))
 (segment (start 189.23 96.52) (end 193.04 100.33) (width 0.8) (layer B.Cu) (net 2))
 (segment (start 185.42 93.98) (end 190.5 93.98) (width 0.8) (layer B.Cu) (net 3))
 (segment (start 190.5 93.98) (end 193.04 91.44) (width 0.8) (layer B.Cu) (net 3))
 (segment (start 193.04 88.9) (end 196.85 88.9) (width 0.8) (layer B.Cu) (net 4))
 (segment (start 187.96 106.68) (end 185.42 104.14) (width 0.8) (layer B.Cu) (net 4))
 (segment (start 198.12 106.68) (end 187.96 106.68) (width 0.8) (layer B.Cu) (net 4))
 (segment (start 199.39 105.41) (end 198.12 106.68) (width 0.8) (layer B.Cu) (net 4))
 (segment (start 199.39 91.44) (end 199.39 105.41) (width 0.8) (layer B.Cu) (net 4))
 (segment (start 196.85 88.9) (end 199.39 91.44) (width 0.8) (layer B.Cu) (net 4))
 (segment (start 185.42 88.9) (end 185.42 86.36) (width 0.8) (layer B.Cu) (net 5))
 (segment (start 185.42 86.36) (end 182.88 83.82) (width 0.8) (layer B.Cu) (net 5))
 (segment (start 182.88 83.82) (end 163.83 83.82) (width 0.8) (layer B.Cu) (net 5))
 (segment (start 168.91 77.47) (end 170.18 77.47) (width 0.8) (layer B.Cu) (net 5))
 (segment (start 163.83 87.48) (end 163.83 93.98) (width 0.8) (layer B.Cu) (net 5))
 (segment (start 153.67 87.48) (end 153.67 93.98) (width 0.8) (layer B.Cu) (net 5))
 (segment (start 163.83 87.48) (end 163.83 83.82) (width 0.8) (layer B.Cu) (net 5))
 (segment (start 163.83 83.82) (end 163.83 82.55) (width 0.8) (layer B.Cu) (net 5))
 (segment (start 163.83 82.55) (end 168.91 77.47) (width 0.8) (layer B.Cu) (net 5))
 (segment (start 153.67 87.48) (end 153.67 82.55) (width 0.8) (layer B.Cu) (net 5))
 (segment (start 158.75 77.47) (end 168.91 77.47) (width 0.8) (layer B.Cu) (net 5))
 (segment (start 168.91 77.47) (end 170.18 77.47) (width 0.8) (layer B.Cu) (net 5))
 (segment (start 170.18 77.47) (end 173.99 77.47) (width 0.8) (layer B.Cu) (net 5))
 (segment (start 153.67 82.55) (end 158.75 77.47) (width 0.8) (layer B.Cu) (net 5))
 (segment (start 168.33 93.98) (end 168.33 87.48) (width 0.8) (layer B.Cu) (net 7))
 (segment (start 168.33 87.48) (end 176.38 87.48) (width 0.8) (layer B.Cu) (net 7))
 (segment (start 176.38 87.48) (end 177.8 88.9) (width 0.8) (layer B.Cu) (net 7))
 (segment (start 158.17 93.98) (end 158.17 95.94) (width 0.8) (layer B.Cu) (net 8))
 (segment (start 172.72 96.52) (end 177.8 91.44) (width 0.8) (layer B.Cu) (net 8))
 (segment (start 158.75 96.52) (end 172.72 96.52) (width 0.8) (layer B.Cu) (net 8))
 (segment (start 158.17 95.94) (end 158.75 96.52) (width 0.8) (layer B.Cu) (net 8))
 (segment (start 182.88 104.14) (end 185.42 101.6) (width 0.8) (layer B.Cu) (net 9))
 (segment (start 182.88 105.41) (end 182.88 104.14) (width 0.8) (layer B.Cu) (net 9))
 (segment (start 180.34 107.95) (end 182.88 105.41) (width 0.8) (layer B.Cu) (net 9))
 (segment (start 177.8 107.95) (end 180.34 107.95) (width 0.8) (layer B.Cu) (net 9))
 (segment (start 175.26 105.41) (end 177.8 107.95) (width 0.8) (layer B.Cu) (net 9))
 (segment (start 175.26 96.52) (end 175.26 105.41) (width 0.8) (layer B.Cu) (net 9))
 (segment (start 177.8 93.98) (end 175.26 96.52) (width 0.8) (layer B.Cu) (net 9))
 (segment (start 177.8 101.6) (end 179.07 101.6) (width 0.8) (layer B.Cu) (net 10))
 (segment (start 179.07 101.6) (end 182.88 97.79) (width 0.8) (layer B.Cu) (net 10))
 (segment (start 182.88 97.79) (end 182.88 93.98) (width 0.8) (layer B.Cu) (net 10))
 (segment (start 182.88 93.98) (end 185.42 91.44) (width 0.8) (layer B.Cu) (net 10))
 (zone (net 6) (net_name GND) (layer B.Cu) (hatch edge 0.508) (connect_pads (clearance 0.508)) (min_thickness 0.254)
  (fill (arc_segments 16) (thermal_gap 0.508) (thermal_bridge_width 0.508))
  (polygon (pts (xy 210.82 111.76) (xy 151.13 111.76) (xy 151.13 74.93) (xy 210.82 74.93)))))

